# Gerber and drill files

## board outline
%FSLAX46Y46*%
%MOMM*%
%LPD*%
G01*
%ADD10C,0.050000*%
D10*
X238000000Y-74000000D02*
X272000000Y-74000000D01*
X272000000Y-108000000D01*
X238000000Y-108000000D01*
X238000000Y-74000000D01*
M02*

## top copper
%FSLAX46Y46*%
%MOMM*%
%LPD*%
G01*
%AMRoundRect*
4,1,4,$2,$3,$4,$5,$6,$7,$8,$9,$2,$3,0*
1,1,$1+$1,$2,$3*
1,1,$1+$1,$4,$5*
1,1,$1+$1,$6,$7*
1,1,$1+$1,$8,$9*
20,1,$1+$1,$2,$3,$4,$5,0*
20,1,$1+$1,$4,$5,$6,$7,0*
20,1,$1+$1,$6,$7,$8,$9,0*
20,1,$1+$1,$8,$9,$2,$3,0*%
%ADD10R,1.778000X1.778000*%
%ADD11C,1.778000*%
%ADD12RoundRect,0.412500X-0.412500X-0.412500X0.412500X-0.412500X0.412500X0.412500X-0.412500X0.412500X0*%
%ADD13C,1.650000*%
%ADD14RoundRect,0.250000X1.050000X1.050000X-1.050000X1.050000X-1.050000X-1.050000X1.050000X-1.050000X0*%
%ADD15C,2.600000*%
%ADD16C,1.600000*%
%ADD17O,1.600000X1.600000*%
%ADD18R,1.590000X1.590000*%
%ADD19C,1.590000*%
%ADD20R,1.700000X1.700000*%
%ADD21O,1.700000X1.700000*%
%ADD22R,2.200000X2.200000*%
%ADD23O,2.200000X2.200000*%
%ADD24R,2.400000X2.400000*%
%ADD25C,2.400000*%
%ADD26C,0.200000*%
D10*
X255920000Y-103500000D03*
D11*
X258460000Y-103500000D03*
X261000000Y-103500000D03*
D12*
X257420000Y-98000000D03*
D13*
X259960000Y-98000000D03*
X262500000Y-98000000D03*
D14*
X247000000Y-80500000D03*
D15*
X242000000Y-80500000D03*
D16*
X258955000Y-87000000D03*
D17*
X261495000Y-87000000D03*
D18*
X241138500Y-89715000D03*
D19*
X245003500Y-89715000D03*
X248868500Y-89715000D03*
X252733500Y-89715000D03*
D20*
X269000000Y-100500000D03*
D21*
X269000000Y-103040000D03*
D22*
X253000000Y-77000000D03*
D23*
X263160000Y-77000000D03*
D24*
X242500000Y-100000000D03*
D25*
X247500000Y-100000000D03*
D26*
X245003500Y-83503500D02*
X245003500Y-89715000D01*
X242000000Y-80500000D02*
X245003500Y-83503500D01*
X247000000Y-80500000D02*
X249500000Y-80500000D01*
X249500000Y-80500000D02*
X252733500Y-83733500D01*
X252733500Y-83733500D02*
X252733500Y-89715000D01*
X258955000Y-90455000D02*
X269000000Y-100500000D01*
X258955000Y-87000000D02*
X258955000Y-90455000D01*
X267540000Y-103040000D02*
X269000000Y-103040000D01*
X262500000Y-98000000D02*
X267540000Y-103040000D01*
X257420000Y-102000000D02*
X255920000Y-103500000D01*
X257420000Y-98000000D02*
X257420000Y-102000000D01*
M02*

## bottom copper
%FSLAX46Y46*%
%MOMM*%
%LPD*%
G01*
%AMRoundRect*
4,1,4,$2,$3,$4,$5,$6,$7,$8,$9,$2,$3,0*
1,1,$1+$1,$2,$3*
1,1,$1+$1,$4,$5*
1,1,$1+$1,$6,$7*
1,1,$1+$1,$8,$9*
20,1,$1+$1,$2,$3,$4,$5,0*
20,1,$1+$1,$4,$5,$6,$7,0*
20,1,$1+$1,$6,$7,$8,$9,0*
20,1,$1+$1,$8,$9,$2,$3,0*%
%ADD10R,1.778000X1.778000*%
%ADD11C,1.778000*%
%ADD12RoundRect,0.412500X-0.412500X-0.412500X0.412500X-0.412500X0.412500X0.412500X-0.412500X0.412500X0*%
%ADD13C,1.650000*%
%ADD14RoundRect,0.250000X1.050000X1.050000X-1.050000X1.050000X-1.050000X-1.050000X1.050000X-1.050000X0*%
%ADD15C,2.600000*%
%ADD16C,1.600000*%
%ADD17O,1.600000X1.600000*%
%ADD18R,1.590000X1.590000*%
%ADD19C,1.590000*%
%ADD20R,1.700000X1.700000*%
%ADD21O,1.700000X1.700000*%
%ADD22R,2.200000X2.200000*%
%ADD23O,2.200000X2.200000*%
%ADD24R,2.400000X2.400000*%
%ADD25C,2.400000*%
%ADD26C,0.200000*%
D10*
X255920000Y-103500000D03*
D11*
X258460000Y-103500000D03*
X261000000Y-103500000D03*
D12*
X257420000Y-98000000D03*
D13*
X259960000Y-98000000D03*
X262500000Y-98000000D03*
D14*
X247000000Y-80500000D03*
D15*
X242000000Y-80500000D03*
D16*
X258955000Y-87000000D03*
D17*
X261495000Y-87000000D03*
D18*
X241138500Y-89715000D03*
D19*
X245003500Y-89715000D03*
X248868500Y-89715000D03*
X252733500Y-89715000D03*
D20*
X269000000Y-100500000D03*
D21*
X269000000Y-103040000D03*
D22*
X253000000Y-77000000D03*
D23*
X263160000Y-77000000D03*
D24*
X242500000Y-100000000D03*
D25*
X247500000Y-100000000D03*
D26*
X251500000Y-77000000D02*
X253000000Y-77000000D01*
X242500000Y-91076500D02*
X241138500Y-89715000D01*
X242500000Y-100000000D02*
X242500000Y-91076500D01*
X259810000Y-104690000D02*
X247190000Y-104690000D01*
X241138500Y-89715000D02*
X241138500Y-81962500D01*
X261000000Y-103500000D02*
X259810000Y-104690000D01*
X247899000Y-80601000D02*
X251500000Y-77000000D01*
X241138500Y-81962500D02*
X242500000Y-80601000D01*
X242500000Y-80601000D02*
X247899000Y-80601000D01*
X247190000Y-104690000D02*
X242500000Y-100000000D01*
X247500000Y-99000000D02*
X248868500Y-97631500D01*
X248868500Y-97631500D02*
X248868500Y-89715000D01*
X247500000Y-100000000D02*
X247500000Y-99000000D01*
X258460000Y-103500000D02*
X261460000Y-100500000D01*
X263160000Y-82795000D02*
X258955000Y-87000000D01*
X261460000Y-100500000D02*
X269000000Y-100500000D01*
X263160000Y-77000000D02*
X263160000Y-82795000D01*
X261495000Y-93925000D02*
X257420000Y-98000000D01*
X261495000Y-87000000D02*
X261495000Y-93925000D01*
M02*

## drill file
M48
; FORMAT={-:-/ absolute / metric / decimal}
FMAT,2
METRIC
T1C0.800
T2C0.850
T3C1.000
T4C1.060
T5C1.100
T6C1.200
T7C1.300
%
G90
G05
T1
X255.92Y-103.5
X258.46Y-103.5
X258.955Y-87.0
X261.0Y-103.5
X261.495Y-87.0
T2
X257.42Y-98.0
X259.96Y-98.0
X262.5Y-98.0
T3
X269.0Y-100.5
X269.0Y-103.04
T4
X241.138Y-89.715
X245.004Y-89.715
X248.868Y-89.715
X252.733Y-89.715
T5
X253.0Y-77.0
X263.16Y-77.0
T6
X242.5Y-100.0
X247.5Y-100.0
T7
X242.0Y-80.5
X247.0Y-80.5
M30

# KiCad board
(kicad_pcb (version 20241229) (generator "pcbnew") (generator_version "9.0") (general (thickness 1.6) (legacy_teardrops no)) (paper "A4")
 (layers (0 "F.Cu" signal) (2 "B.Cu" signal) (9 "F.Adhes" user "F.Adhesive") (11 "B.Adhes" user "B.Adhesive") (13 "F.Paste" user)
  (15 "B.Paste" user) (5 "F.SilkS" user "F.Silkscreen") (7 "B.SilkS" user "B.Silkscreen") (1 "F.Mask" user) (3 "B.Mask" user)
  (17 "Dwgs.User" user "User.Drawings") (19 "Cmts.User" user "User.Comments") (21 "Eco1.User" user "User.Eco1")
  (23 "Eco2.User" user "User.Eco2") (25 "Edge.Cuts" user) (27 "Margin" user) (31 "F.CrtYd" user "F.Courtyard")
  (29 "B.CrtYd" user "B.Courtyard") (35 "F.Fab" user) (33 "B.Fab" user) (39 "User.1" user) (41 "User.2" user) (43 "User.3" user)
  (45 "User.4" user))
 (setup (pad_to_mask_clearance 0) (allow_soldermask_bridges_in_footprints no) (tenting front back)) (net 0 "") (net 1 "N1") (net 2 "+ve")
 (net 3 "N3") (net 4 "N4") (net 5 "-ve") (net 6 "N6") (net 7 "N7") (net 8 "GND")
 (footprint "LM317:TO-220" (layer "F.Cu") (at 258.46 103.5)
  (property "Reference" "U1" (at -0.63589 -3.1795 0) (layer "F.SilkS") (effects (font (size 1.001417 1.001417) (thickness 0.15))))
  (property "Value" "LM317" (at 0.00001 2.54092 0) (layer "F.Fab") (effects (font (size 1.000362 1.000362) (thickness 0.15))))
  (pad "1" thru_hole rect (at -2.54 0) (size 1.778 1.778) (drill 0.8) (layers "*.Cu" "*.Mask") (remove_unused_layers no) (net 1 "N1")
   (solder_mask_margin 0.102))
  (pad "2" thru_hole circle (at 0 0) (size 1.778 1.778) (drill 0.8) (layers "*.Cu" "*.Mask") (remove_unused_layers no) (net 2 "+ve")
   (solder_mask_margin 0.102))
  (pad "3" thru_hole circle (at 2.54 0) (size 1.778 1.778) (drill 0.8) (layers "*.Cu" "*.Mask") (remove_unused_layers no) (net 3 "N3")
   (solder_mask_margin 0.102)))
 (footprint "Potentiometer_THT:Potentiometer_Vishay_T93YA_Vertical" (layer "F.Cu") (at 257.42 98)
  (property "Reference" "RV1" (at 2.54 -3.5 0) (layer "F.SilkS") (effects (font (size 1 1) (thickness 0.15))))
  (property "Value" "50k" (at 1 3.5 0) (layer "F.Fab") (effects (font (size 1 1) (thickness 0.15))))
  (pad "1" thru_hole roundrect (at 0 0) (size 1.65 1.65) (drill 0.85) (layers "*.Cu" "*.Mask") (remove_unused_layers no)
   (roundrect_rratio 0.25) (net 1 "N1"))
  (pad "2" thru_hole circle (at 2.54 0) (size 1.65 1.65) (drill 0.85) (layers "*.Cu" "*.Mask") (remove_unused_layers no) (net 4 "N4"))
  (pad "3" thru_hole circle (at 5.08 0) (size 1.65 1.65) (drill 0.85) (layers "*.Cu" "*.Mask") (remove_unused_layers no) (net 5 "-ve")))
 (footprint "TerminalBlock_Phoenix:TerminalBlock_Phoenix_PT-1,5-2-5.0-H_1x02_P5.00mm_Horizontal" (layer "F.Cu") (at 247 80.5 180)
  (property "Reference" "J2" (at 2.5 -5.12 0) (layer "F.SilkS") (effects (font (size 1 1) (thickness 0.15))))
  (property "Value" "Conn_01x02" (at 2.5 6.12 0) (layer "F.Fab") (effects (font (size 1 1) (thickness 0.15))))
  (pad "1" thru_hole roundrect (at 0 0 180) (size 2.6 2.6) (drill 1.3) (layers "*.Cu" "*.Mask") (remove_unused_layers no)
   (roundrect_rratio 0.096154) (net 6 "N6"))
  (pad "2" thru_hole circle (at 5 0 180) (size 2.6 2.6) (drill 1.3) (layers "*.Cu" "*.Mask") (remove_unused_layers no) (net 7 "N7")))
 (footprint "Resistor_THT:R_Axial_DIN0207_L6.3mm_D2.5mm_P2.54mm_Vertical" (layer "F.Cu") (at 258.955 87)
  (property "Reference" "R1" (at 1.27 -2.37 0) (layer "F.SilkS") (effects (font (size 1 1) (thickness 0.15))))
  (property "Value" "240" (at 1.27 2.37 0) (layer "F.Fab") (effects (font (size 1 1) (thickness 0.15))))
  (pad "1" thru_hole circle (at 0 0) (size 1.6 1.6) (drill 0.8) (layers "*.Cu" "*.Mask") (remove_unused_layers no) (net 2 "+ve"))
  (pad "2" thru_hole oval (at 2.54 0) (size 1.6 1.6) (drill 0.8) (layers "*.Cu" "*.Mask") (remove_unused_layers no) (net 1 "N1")))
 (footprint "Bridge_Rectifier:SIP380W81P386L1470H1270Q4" (layer "F.Cu") (at 241.1385 89.715)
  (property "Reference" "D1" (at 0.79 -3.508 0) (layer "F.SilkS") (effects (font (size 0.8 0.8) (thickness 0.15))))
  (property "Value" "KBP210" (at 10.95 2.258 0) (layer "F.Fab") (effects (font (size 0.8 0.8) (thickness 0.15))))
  (pad "1" thru_hole rect (at 0 0) (size 1.59 1.59) (drill 1.06) (layers "*.Cu" "*.Mask") (remove_unused_layers no) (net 3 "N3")
   (solder_mask_margin 0.102))
  (pad "2" thru_hole circle (at 3.865 0) (size 1.59 1.59) (drill 1.06) (layers "*.Cu" "*.Mask") (remove_unused_layers no) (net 7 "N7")
   (solder_mask_margin 0.102))
  (pad "3" thru_hole circle (at 7.73 0) (size 1.59 1.59) (drill 1.06) (layers "*.Cu" "*.Mask") (remove_unused_layers no) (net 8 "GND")
   (solder_mask_margin 0.102))
  (pad "4" thru_hole circle (at 11.595 0) (size 1.59 1.59) (drill 1.06) (layers "*.Cu" "*.Mask") (remove_unused_layers no) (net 6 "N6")
   (solder_mask_margin 0.102)))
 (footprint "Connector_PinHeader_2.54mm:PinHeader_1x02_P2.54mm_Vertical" (layer "F.Cu") (at 269 100.5)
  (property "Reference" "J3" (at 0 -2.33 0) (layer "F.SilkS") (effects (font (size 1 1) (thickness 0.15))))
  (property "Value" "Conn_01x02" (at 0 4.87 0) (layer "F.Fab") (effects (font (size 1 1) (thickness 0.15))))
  (pad "1" thru_hole rect (at 0 0) (size 1.7 1.7) (drill 1) (layers "*.Cu" "*.Mask") (remove_unused_layers no) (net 2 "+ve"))
  (pad "2" thru_hole oval (at 0 2.54) (size 1.7 1.7) (drill 1) (layers "*.Cu" "*.Mask") (remove_unused_layers no) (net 5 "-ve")))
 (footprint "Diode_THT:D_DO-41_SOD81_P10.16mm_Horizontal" (layer "F.Cu") (at 253 77)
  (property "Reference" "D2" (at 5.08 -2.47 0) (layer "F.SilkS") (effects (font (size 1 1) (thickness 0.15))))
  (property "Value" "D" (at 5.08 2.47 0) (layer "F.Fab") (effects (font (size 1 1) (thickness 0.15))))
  (pad "1" thru_hole rect (at 0 0) (size 2.2 2.2) (drill 1.1) (layers "*.Cu" "*.Mask") (remove_unused_layers no) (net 3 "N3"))
  (pad "2" thru_hole oval (at 10.16 0) (size 2.2 2.2) (drill 1.1) (layers "*.Cu" "*.Mask") (remove_unused_layers no) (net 2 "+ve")))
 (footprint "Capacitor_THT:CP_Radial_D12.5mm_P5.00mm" (layer "F.Cu") (at 242.5 100)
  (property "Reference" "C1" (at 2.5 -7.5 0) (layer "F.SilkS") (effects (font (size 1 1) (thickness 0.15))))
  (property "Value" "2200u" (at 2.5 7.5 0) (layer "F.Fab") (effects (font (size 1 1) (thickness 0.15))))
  (pad "1" thru_hole rect (at 0 0) (size 2.4 2.4) (drill 1.2) (layers "*.Cu" "*.Mask") (remove_unused_layers no) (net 3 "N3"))
  (pad "2" thru_hole circle (at 5 0) (size 2.4 2.4) (drill 1.2) (layers "*.Cu" "*.Mask") (remove_unused_layers no) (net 8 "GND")))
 (gr_rect (start 238 74) (end 272 108) (stroke (width 0.05) (type default)) (fill no) (layer "Edge.Cuts"))
 (segment (start 251.5 77) (end 253 77) (width 0.2) (layer "B.Cu") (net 3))
 (segment (start 242.5 91.0765) (end 241.1385 89.715) (width 0.2) (layer "B.Cu") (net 3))
 (segment (start 242.5 100) (end 242.5 91.0765) (width 0.2) (layer "B.Cu") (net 3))
 (segment (start 259.81 104.69) (end 247.19 104.69) (width 0.2) (layer "B.Cu") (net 3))
 (segment (start 241.1385 89.715) (end 241.1385 81.9625) (width 0.2) (layer "B.Cu") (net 3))
 (segment (start 261 103.5) (end 259.81 104.69) (width 0.2) (layer "B.Cu") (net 3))
 (segment (start 247.899 80.601) (end 251.5 77) (width 0.2) (layer "B.Cu") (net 3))
 (segment (start 241.1385 81.9625) (end 242.5 80.601) (width 0.2) (layer "B.Cu") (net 3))
 (segment (start 242.5 80.601) (end 247.899 80.601) (width 0.2) (layer "B.Cu") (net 3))
 (segment (start 247.19 104.69) (end 242.5 100) (width 0.2) (layer "B.Cu") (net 3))
 (segment (start 247.5 99) (end 248.8685 97.6315) (width 0.2) (layer "B.Cu") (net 8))
 (segment (start 248.8685 97.6315) (end 248.8685 89.715) (width 0.2) (layer "B.Cu") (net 8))
 (segment (start 247.5 100) (end 247.5 99) (width 0.2) (layer "B.Cu") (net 8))
 (segment (start 245.0035 83.5035) (end 245.0035 89.715) (width 0.2) (layer "F.Cu") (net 7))
 (segment (start 242 80.5) (end 245.0035 83.5035) (width 0.2) (layer "F.Cu") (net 7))
 (segment (start 247 80.5) (end 249.5 80.5) (width 0.2) (layer "F.Cu") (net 6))
 (segment (start 249.5 80.5) (end 252.7335 83.7335) (width 0.2) (layer "F.Cu") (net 6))
 (segment (start 252.7335 83.7335) (end 252.7335 89.715) (width 0.2) (layer "F.Cu") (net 6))
 (segment (start 258.955 90.455) (end 269 100.5) (width 0.2) (layer "F.Cu") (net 2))
 (segment (start 258.955 87) (end 258.955 90.455) (width 0.2) (layer "F.Cu") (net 2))
 (segment (start 258.46 103.5) (end 261.46 100.5) (width 0.2) (layer "B.Cu") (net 2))
 (segment (start 263.16 82.795) (end 258.955 87) (width 0.2) (layer "B.Cu") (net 2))
 (segment (start 261.46 100.5) (end 269 100.5) (width 0.2) (layer "B.Cu") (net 2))
 (segment (start 263.16 77) (end 263.16 82.795) (width 0.2) (layer "B.Cu") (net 2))
 (segment (start 267.54 103.04) (end 269 103.04) (width 0.2) (layer "F.Cu") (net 5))
 (segment (start 262.5 98) (end 267.54 103.04) (width 0.2) (layer "F.Cu") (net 5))
 (segment (start 257.42 102) (end 255.92 103.5) (width 0.2) (layer "F.Cu") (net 1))
 (segment (start 257.42 98) (end 257.42 102) (width 0.2) (layer "F.Cu") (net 1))
 (segment (start 261.495 93.925) (end 257.42 98) (width 0.2) (layer "B.Cu") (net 1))
 (segment (start 261.495 87) (end 261.495 93.925) (width 0.2) (layer "B.Cu") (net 1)))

